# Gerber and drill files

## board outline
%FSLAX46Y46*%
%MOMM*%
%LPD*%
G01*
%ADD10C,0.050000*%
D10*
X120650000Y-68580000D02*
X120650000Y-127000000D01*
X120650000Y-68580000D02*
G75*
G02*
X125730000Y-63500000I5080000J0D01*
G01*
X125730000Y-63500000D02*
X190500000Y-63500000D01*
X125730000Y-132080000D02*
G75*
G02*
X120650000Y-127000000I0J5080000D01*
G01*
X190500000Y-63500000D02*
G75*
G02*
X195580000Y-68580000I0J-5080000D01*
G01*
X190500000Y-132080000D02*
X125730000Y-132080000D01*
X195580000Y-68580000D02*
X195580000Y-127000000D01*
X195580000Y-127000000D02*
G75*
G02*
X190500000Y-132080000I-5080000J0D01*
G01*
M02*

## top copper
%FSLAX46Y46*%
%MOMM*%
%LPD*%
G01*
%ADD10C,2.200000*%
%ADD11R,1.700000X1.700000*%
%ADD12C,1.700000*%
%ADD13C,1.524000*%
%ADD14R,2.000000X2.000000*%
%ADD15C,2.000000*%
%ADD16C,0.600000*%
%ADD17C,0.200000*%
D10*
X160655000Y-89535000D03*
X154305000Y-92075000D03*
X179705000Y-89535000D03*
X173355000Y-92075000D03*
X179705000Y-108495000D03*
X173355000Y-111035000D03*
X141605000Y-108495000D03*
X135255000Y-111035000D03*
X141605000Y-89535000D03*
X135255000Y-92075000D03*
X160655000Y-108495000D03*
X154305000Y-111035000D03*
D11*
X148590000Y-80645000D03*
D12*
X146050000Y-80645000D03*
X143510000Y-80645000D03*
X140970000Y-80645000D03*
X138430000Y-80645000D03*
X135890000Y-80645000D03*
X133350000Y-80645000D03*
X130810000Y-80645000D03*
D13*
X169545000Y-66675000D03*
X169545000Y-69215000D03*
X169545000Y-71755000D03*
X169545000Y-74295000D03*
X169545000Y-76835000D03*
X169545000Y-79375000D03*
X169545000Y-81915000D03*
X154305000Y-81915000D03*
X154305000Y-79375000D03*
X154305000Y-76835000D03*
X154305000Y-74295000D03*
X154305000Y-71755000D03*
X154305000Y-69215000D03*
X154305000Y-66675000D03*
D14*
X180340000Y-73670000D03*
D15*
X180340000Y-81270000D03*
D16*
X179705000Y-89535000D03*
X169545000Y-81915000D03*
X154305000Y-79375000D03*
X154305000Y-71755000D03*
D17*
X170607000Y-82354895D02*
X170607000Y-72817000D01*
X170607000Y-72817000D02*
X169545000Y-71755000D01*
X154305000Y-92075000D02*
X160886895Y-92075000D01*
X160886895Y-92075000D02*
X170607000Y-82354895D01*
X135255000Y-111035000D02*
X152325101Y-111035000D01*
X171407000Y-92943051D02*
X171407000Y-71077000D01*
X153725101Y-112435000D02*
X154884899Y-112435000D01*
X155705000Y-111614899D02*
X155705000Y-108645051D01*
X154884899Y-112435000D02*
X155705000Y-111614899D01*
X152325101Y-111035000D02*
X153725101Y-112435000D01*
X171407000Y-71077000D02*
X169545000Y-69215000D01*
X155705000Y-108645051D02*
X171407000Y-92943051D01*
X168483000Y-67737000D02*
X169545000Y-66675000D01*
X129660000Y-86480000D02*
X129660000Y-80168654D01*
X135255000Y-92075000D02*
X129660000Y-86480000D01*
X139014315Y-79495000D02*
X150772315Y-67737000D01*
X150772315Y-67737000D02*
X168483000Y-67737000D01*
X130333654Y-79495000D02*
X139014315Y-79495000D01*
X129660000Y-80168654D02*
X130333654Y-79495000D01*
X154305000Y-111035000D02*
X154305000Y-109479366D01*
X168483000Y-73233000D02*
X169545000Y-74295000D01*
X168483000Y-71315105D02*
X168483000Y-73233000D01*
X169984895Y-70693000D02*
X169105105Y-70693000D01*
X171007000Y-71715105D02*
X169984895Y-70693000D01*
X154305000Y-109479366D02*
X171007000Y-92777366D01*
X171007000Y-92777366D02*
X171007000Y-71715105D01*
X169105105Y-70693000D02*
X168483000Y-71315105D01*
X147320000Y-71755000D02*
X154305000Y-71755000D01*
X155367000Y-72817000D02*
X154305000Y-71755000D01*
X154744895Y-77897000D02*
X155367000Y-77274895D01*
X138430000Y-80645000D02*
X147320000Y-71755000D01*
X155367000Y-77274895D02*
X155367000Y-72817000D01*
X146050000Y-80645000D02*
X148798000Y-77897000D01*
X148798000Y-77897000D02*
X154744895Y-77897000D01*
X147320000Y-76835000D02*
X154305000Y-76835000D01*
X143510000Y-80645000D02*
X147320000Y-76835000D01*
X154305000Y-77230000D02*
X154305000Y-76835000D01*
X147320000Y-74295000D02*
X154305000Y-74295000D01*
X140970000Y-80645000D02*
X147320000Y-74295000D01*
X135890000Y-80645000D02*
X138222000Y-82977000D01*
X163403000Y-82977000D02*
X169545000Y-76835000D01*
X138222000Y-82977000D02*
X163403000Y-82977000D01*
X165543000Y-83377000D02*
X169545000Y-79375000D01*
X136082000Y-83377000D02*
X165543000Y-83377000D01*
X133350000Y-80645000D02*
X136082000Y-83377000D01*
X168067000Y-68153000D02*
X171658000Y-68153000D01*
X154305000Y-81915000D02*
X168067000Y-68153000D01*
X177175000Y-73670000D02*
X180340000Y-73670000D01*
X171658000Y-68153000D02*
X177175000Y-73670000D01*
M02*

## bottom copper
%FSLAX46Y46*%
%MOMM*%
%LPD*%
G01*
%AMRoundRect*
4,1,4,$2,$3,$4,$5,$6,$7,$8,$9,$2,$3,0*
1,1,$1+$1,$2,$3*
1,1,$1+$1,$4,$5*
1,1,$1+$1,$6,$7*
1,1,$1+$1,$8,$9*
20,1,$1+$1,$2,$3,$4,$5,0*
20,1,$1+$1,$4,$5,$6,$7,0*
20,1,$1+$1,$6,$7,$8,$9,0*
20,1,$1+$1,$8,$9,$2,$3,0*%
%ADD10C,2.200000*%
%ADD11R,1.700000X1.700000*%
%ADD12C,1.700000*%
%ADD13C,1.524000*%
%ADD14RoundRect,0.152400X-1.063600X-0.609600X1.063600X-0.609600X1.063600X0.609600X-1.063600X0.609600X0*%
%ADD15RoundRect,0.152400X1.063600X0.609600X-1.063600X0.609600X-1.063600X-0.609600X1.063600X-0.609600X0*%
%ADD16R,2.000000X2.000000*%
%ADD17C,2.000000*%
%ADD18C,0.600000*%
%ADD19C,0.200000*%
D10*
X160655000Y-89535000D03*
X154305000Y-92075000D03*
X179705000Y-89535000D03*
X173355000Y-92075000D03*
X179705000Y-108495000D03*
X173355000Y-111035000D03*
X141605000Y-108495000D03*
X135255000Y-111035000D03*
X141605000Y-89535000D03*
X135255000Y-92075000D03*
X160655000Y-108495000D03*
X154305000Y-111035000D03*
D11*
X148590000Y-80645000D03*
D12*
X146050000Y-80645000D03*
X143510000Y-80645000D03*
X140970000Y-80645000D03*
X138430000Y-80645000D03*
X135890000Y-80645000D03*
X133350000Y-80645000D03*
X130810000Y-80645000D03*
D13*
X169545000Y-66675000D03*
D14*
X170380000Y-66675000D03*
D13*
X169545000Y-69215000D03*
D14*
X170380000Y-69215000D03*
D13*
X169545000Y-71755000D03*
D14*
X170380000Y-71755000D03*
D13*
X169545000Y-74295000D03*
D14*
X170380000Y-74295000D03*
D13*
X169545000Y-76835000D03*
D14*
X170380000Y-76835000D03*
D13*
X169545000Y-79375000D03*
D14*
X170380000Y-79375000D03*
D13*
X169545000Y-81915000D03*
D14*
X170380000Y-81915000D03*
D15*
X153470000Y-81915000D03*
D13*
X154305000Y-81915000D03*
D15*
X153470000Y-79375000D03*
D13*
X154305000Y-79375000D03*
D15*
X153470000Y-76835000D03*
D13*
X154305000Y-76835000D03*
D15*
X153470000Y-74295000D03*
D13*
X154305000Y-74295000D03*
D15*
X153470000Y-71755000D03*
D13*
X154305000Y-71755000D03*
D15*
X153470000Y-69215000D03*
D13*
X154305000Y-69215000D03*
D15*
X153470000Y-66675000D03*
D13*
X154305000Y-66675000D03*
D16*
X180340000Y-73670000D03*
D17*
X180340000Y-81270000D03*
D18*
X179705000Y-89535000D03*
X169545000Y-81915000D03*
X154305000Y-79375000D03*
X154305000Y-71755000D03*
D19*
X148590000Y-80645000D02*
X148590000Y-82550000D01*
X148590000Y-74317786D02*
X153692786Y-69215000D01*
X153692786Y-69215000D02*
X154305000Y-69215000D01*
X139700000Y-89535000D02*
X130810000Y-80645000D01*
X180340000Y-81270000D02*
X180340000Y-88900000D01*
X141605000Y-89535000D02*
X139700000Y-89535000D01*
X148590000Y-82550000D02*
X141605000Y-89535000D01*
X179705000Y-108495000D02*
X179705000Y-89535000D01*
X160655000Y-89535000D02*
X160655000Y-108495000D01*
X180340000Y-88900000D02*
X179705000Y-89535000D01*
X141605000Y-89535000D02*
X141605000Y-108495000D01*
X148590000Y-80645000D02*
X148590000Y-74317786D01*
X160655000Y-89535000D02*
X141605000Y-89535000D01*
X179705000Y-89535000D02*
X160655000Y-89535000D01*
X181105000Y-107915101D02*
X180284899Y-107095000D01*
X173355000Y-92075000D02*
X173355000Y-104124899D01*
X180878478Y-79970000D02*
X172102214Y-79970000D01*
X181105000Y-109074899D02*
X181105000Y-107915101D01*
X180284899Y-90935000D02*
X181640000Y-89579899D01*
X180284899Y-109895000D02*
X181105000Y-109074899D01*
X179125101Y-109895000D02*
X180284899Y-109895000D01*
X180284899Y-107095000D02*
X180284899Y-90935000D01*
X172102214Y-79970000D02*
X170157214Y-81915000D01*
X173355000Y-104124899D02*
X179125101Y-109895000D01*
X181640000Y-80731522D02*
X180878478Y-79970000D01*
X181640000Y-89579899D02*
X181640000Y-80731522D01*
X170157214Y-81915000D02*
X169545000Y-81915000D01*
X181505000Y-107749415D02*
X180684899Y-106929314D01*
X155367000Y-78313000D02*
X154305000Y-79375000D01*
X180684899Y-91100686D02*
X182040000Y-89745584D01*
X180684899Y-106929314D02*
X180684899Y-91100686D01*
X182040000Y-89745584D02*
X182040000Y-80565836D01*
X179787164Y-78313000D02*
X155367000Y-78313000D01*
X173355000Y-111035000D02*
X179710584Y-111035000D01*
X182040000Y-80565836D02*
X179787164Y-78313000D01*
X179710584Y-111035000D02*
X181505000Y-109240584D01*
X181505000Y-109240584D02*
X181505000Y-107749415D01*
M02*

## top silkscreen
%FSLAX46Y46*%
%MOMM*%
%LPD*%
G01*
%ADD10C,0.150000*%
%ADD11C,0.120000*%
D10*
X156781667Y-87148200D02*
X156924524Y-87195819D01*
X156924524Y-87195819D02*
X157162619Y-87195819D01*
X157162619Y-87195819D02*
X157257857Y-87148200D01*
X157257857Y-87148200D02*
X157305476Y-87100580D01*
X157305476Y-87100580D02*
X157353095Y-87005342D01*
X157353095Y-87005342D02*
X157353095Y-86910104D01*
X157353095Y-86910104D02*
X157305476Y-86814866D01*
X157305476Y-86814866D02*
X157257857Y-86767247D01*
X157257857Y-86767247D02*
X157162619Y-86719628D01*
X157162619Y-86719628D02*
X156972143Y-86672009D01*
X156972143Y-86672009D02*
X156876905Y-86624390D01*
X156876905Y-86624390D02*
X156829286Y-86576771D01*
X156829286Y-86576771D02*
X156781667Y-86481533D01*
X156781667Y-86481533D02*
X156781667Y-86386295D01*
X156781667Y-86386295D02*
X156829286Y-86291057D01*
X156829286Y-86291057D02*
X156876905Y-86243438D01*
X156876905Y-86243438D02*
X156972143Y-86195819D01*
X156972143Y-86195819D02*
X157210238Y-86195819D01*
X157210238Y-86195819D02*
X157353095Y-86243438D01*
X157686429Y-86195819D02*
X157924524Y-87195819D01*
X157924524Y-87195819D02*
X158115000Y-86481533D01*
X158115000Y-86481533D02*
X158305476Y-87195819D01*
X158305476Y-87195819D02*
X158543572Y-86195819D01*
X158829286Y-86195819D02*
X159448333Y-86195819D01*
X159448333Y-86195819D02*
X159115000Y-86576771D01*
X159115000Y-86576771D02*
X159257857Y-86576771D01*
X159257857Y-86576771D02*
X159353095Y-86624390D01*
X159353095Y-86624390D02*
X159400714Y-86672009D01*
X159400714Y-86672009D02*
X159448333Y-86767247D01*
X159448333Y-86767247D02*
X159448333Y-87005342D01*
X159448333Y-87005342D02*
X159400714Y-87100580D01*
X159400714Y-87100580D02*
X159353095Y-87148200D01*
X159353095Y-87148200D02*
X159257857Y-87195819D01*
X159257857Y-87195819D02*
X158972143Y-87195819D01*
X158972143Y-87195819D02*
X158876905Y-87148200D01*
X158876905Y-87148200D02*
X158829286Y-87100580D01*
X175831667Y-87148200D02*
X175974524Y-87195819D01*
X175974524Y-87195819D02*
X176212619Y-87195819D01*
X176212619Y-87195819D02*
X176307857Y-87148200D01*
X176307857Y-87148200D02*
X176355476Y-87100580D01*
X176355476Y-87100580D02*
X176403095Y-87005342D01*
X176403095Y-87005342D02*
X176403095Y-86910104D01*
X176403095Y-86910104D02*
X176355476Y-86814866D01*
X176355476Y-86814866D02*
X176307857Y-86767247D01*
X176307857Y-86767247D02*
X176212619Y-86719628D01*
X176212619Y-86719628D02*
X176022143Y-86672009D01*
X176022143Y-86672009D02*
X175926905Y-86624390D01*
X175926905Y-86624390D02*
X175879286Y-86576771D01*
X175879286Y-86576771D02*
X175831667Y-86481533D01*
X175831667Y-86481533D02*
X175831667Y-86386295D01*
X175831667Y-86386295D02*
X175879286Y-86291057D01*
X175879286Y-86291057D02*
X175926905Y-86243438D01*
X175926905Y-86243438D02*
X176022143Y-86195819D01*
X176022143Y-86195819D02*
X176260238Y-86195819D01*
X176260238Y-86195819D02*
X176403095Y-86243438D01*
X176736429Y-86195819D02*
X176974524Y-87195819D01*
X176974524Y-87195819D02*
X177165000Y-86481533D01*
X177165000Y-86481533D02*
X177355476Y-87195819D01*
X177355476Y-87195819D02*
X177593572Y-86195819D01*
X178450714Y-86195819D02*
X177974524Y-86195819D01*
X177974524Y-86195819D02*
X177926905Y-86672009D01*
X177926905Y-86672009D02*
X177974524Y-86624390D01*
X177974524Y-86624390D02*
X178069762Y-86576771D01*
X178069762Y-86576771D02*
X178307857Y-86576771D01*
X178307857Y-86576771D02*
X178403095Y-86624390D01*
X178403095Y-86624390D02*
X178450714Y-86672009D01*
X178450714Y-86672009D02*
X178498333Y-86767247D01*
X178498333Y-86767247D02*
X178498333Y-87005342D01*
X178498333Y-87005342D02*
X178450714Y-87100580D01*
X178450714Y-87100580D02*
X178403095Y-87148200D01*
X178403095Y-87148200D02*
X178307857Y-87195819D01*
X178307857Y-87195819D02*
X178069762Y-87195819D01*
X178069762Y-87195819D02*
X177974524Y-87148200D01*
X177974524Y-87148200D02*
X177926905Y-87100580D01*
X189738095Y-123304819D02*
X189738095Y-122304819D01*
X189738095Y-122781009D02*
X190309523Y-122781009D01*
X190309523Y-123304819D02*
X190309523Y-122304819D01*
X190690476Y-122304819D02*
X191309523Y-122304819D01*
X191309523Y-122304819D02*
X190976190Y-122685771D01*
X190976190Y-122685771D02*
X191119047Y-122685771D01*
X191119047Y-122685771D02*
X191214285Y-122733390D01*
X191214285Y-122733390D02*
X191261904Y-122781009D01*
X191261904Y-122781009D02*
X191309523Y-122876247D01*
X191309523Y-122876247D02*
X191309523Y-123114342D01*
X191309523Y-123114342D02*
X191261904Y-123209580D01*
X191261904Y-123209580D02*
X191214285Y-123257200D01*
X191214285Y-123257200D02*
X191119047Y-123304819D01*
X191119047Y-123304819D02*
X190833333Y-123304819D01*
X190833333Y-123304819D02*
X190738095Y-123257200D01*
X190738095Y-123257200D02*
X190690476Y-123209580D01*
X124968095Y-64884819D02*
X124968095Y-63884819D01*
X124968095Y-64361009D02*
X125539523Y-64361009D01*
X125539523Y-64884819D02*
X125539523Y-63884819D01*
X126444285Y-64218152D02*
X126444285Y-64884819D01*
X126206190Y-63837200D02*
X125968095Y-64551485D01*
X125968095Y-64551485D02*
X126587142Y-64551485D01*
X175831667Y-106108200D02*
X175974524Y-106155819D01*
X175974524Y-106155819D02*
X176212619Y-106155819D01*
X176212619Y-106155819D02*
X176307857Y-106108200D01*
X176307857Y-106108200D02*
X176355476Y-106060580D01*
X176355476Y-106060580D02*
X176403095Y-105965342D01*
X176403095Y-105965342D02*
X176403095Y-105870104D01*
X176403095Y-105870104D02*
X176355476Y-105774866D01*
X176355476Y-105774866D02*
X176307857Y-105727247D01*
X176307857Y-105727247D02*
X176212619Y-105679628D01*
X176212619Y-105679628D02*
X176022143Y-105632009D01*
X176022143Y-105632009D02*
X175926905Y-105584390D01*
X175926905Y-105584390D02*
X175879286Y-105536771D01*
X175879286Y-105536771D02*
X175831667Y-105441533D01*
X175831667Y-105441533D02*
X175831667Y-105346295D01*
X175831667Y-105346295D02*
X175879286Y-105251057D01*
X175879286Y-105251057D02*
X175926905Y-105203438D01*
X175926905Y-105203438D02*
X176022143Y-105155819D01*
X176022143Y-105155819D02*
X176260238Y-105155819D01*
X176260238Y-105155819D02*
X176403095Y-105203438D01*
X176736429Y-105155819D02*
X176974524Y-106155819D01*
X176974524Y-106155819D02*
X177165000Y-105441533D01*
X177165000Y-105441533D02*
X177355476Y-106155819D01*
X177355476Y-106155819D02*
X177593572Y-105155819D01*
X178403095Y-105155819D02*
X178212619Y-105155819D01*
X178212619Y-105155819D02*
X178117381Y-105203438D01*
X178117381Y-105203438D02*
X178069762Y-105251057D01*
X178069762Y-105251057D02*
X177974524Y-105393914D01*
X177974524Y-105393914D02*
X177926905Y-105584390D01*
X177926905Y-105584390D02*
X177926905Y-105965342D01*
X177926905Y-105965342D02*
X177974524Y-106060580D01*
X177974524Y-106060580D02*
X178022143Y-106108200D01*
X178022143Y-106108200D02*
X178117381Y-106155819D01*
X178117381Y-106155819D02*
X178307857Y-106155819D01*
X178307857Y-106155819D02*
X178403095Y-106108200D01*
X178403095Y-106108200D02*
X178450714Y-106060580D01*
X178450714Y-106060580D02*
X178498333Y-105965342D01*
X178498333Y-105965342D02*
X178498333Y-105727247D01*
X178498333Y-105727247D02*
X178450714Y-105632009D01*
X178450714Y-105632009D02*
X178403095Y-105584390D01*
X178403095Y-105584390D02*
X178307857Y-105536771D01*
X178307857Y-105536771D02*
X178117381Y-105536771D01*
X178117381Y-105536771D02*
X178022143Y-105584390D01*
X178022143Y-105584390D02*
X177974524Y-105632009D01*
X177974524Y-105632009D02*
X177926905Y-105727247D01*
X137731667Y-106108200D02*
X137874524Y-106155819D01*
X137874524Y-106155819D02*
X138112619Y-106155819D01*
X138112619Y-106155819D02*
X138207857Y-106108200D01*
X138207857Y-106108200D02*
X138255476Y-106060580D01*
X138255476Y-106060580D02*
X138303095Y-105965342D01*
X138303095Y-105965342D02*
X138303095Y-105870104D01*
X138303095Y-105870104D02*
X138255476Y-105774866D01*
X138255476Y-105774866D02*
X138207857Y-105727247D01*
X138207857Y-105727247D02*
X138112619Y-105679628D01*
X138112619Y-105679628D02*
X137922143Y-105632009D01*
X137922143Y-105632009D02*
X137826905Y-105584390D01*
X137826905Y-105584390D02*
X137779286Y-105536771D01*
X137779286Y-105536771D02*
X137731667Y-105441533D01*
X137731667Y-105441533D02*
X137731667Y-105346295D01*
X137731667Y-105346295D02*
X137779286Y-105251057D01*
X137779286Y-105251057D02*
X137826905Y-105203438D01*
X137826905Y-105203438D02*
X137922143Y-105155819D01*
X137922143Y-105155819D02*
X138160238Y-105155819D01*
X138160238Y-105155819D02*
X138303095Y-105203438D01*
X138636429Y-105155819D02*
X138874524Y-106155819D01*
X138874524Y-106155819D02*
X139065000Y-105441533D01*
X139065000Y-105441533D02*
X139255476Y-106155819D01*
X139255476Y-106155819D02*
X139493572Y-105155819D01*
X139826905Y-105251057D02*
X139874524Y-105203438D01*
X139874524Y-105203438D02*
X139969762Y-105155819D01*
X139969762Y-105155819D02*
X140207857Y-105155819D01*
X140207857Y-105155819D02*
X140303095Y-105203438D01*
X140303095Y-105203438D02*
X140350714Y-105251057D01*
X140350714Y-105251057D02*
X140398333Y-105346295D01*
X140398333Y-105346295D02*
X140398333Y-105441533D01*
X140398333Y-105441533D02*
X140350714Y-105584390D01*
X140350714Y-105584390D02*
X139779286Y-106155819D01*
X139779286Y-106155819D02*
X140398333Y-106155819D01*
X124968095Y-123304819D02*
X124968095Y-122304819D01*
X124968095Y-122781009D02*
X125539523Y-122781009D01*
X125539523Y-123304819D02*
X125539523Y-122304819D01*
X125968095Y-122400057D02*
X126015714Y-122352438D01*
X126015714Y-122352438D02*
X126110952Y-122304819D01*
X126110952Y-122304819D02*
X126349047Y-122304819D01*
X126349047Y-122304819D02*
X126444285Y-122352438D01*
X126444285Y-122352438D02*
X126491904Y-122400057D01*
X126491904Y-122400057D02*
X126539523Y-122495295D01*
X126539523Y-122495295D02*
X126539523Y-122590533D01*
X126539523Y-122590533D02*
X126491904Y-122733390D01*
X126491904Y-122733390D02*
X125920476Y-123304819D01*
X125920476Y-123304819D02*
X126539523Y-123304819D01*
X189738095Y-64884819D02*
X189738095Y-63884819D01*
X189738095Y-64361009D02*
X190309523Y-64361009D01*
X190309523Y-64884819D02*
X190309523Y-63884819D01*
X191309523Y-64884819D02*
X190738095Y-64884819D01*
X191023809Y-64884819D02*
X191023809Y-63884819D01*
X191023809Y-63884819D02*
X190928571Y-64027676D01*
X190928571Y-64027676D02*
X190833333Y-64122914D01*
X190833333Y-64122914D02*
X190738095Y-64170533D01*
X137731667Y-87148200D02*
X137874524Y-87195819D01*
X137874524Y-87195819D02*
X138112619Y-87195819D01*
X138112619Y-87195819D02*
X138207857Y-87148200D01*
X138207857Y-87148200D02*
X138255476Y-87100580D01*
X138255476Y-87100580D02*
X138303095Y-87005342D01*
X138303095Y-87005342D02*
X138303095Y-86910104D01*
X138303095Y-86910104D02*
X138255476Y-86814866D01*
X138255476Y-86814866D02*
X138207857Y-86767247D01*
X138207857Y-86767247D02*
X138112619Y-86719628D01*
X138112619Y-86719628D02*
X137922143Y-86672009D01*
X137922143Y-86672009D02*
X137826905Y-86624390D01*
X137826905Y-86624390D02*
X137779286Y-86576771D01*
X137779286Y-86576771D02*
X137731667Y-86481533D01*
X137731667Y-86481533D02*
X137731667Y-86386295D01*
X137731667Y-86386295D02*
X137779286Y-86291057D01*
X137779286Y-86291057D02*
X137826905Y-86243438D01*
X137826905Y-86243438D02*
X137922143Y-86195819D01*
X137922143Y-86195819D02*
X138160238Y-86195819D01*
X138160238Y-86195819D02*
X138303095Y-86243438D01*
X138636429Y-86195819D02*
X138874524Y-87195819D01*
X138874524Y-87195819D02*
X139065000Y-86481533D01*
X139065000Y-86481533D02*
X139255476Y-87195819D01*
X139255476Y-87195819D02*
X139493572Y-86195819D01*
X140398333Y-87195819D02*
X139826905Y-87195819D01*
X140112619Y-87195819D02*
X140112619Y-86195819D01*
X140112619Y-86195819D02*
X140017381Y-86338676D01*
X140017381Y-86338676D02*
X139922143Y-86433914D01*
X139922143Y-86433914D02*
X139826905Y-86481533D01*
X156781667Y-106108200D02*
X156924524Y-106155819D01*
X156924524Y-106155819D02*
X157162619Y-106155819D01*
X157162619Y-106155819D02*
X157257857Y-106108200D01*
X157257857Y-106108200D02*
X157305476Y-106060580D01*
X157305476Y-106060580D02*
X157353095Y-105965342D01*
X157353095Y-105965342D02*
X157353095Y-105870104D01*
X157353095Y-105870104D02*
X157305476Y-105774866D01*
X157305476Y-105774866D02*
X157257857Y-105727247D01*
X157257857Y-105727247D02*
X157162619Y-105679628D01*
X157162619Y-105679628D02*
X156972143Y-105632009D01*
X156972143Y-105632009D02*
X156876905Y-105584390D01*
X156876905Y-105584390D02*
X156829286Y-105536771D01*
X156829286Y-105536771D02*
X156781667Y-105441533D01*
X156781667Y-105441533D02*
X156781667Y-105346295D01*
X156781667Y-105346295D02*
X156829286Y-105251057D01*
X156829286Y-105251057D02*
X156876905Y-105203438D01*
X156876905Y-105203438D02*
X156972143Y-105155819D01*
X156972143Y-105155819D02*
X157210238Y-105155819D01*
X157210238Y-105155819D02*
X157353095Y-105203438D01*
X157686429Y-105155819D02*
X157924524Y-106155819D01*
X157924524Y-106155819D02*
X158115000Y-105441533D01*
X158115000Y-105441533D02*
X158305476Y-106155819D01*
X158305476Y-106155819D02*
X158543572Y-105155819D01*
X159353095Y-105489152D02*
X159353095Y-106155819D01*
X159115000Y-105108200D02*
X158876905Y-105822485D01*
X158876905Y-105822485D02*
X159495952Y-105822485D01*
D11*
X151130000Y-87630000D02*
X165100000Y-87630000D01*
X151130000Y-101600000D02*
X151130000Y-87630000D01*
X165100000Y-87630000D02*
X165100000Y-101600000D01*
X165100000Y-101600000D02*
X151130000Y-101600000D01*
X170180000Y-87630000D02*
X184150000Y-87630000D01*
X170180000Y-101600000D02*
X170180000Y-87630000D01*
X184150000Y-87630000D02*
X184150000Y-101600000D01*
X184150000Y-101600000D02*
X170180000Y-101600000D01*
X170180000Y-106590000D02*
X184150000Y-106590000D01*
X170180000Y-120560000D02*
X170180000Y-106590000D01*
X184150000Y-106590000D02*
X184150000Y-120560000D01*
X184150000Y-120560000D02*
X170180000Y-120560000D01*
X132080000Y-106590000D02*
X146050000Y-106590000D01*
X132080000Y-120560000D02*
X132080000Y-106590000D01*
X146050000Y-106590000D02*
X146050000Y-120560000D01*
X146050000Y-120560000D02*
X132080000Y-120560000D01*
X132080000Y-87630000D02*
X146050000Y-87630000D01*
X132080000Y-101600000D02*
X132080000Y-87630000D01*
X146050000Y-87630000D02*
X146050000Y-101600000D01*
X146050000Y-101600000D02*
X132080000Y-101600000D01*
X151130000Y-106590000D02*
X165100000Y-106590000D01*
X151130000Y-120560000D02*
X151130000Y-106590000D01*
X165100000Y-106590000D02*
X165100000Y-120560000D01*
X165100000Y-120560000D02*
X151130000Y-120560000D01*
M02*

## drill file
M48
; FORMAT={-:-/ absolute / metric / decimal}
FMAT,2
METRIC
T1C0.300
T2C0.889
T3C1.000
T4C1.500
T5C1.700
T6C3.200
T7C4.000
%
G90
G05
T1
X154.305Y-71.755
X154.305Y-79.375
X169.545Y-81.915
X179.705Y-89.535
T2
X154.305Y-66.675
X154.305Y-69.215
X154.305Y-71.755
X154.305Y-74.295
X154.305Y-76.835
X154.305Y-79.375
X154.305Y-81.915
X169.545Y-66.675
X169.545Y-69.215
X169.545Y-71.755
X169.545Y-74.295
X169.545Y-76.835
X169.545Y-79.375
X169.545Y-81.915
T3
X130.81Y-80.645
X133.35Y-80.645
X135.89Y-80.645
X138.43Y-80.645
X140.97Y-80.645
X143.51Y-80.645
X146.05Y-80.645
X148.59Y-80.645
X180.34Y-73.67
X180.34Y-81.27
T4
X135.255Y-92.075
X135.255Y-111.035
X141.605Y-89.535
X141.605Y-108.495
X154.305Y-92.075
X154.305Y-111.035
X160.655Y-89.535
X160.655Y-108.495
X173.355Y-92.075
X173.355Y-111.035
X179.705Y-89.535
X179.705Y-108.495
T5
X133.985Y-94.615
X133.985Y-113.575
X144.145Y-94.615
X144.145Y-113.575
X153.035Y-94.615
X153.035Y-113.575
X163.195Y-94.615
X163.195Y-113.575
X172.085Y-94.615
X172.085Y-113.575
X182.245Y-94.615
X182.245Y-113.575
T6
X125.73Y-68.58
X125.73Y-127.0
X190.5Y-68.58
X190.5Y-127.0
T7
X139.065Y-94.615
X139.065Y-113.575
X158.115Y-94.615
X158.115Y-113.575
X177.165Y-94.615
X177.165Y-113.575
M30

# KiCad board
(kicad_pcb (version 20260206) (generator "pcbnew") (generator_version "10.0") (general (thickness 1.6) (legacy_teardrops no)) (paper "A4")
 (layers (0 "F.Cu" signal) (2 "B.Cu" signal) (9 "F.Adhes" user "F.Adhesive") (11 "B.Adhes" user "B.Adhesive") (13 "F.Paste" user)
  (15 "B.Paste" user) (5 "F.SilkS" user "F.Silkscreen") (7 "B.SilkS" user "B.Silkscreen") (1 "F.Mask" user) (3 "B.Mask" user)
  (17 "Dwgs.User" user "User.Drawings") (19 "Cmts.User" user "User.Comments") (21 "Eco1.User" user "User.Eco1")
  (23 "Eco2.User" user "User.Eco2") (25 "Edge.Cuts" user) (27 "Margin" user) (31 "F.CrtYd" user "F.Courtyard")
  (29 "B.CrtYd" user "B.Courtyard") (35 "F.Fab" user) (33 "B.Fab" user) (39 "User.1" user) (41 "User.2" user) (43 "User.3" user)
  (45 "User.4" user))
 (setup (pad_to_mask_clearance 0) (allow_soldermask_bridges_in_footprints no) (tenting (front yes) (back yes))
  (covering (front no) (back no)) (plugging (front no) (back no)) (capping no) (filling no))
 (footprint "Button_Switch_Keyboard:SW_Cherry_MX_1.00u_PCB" (layer "F.Cu") (at 160.655 89.535)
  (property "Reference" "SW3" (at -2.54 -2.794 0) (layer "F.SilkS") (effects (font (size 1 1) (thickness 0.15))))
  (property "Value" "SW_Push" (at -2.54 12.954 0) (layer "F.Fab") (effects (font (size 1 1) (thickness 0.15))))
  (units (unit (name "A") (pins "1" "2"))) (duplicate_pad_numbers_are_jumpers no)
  (fp_line (start -9.525 -1.905) (end 4.445 -1.905) (stroke (width 0.12) (type solid)) (layer "F.SilkS"))
  (fp_line (start -9.525 12.065) (end -9.525 -1.905) (stroke (width 0.12) (type solid)) (layer "F.SilkS"))
  (fp_line (start 4.445 -1.905) (end 4.445 12.065) (stroke (width 0.12) (type solid)) (layer "F.SilkS"))
  (fp_line (start 4.445 12.065) (end -9.525 12.065) (stroke (width 0.12) (type solid)) (layer "F.SilkS"))
  (pad "" np_thru_hole circle (at -7.62 5.08) (size 1.7 1.7) (drill 1.7) (layers "*.Cu" "*.Mask"))
  (pad "" np_thru_hole circle (at -2.54 5.08) (size 4 4) (drill 4) (layers "*.Cu" "*.Mask"))
  (pad "" np_thru_hole circle (at 2.54 5.08) (size 1.7 1.7) (drill 1.7) (layers "*.Cu" "*.Mask"))
  (pad "1" thru_hole circle (at 0 0) (size 2.2 2.2) (drill 1.5) (layers "*.Cu" "*.Mask") (remove_unused_layers no) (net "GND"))
  (pad "2" thru_hole circle (at -6.35 2.54) (size 2.2 2.2) (drill 1.5) (layers "*.Cu" "*.Mask") (remove_unused_layers no)
   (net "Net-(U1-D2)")))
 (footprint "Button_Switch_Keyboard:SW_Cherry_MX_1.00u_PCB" (layer "F.Cu") (at 179.705 89.535)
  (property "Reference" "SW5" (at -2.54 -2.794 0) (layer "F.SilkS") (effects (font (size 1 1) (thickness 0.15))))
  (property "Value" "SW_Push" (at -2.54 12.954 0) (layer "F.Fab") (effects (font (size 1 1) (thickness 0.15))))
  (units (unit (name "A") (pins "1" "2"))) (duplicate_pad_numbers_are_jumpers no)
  (fp_line (start -9.525 -1.905) (end 4.445 -1.905) (stroke (width 0.12) (type solid)) (layer "F.SilkS"))
  (fp_line (start -9.525 12.065) (end -9.525 -1.905) (stroke (width 0.12) (type solid)) (layer "F.SilkS"))
  (fp_line (start 4.445 -1.905) (end 4.445 12.065) (stroke (width 0.12) (type solid)) (layer "F.SilkS"))
  (fp_line (start 4.445 12.065) (end -9.525 12.065) (stroke (width 0.12) (type solid)) (layer "F.SilkS"))
  (pad "" np_thru_hole circle (at -7.62 5.08) (size 1.7 1.7) (drill 1.7) (layers "*.Cu" "*.Mask"))
  (pad "" np_thru_hole circle (at -2.54 5.08) (size 4 4) (drill 4) (layers "*.Cu" "*.Mask"))
  (pad "" np_thru_hole circle (at 2.54 5.08) (size 1.7 1.7) (drill 1.7) (layers "*.Cu" "*.Mask"))
  (pad "1" thru_hole circle (at 0 0) (size 2.2 2.2) (drill 1.5) (layers "*.Cu" "*.Mask") (remove_unused_layers no) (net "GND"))
  (pad "2" thru_hole circle (at -6.35 2.54) (size 2.2 2.2) (drill 1.5) (layers "*.Cu" "*.Mask") (remove_unused_layers no)
   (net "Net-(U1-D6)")))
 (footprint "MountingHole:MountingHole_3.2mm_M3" (layer "F.Cu") (at 190.5 127)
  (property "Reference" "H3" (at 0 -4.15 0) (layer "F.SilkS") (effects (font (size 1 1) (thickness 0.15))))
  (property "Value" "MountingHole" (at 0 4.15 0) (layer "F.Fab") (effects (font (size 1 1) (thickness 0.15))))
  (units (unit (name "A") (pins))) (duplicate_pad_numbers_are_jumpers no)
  (pad "" np_thru_hole circle (at 0 0) (size 3.2 3.2) (drill 3.2) (layers "*.Cu" "*.Mask")))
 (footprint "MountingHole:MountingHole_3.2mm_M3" (layer "F.Cu") (at 125.73 68.58)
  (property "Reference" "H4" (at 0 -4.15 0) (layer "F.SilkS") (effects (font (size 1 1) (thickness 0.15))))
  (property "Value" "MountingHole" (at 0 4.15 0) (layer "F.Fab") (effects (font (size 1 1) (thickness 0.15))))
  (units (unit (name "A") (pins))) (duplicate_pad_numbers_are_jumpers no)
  (pad "" np_thru_hole circle (at 0 0) (size 3.2 3.2) (drill 3.2) (layers "*.Cu" "*.Mask")))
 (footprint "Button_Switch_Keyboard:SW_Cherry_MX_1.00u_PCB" (layer "F.Cu") (at 179.705 108.495)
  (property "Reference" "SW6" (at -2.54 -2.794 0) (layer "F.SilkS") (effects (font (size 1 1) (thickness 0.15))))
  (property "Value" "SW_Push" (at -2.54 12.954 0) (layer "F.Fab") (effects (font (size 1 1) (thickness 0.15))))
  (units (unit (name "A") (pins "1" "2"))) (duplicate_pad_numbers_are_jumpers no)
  (fp_line (start -9.525 -1.905) (end 4.445 -1.905) (stroke (width 0.12) (type solid)) (layer "F.SilkS"))
  (fp_line (start -9.525 12.065) (end -9.525 -1.905) (stroke (width 0.12) (type solid)) (layer "F.SilkS"))
  (fp_line (start 4.445 -1.905) (end 4.445 12.065) (stroke (width 0.12) (type solid)) (layer "F.SilkS"))
  (fp_line (start 4.445 12.065) (end -9.525 12.065) (stroke (width 0.12) (type solid)) (layer "F.SilkS"))
  (pad "" np_thru_hole circle (at -7.62 5.08) (size 1.7 1.7) (drill 1.7) (layers "*.Cu" "*.Mask"))
  (pad "" np_thru_hole circle (at -2.54 5.08) (size 4 4) (drill 4) (layers "*.Cu" "*.Mask"))
  (pad "" np_thru_hole circle (at 2.54 5.08) (size 1.7 1.7) (drill 1.7) (layers "*.Cu" "*.Mask"))
  (pad "1" thru_hole circle (at 0 0) (size 2.2 2.2) (drill 1.5) (layers "*.Cu" "*.Mask") (remove_unused_layers no) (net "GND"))
  (pad "2" thru_hole circle (at -6.35 2.54) (size 2.2 2.2) (drill 1.5) (layers "*.Cu" "*.Mask") (remove_unused_layers no)
   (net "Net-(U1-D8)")))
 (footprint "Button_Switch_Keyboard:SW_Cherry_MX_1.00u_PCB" (layer "F.Cu") (at 141.605 108.495)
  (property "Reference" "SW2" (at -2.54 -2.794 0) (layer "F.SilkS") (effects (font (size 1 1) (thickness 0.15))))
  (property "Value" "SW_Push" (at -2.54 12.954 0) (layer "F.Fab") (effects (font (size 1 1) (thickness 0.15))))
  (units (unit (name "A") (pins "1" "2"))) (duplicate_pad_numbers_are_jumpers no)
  (fp_line (start -9.525 -1.905) (end 4.445 -1.905) (stroke (width 0.12) (type solid)) (layer "F.SilkS"))
  (fp_line (start -9.525 12.065) (end -9.525 -1.905) (stroke (width 0.12) (type solid)) (layer "F.SilkS"))
  (fp_line (start 4.445 -1.905) (end 4.445 12.065) (stroke (width 0.12) (type solid)) (layer "F.SilkS"))
  (fp_line (start 4.445 12.065) (end -9.525 12.065) (stroke (width 0.12) (type solid)) (layer "F.SilkS"))
  (pad "" np_thru_hole circle (at -7.62 5.08) (size 1.7 1.7) (drill 1.7) (layers "*.Cu" "*.Mask"))
  (pad "" np_thru_hole circle (at -2.54 5.08) (size 4 4) (drill 4) (layers "*.Cu" "*.Mask"))
  (pad "" np_thru_hole circle (at 2.54 5.08) (size 1.7 1.7) (drill 1.7) (layers "*.Cu" "*.Mask"))
  (pad "1" thru_hole circle (at 0 0) (size 2.2 2.2) (drill 1.5) (layers "*.Cu" "*.Mask") (remove_unused_layers no) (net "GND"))
  (pad "2" thru_hole circle (at -6.35 2.54) (size 2.2 2.2) (drill 1.5) (layers "*.Cu" "*.Mask") (remove_unused_layers no)
   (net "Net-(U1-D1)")))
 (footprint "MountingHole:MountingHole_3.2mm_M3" (layer "F.Cu") (at 125.73 127)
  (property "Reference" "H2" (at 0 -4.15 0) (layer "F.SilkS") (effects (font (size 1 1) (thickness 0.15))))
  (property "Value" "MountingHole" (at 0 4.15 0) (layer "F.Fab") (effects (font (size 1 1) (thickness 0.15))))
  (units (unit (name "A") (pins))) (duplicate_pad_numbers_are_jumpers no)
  (pad "" np_thru_hole circle (at 0 0) (size 3.2 3.2) (drill 3.2) (layers "*.Cu" "*.Mask")))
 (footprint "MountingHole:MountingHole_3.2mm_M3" (layer "F.Cu") (at 190.5 68.58)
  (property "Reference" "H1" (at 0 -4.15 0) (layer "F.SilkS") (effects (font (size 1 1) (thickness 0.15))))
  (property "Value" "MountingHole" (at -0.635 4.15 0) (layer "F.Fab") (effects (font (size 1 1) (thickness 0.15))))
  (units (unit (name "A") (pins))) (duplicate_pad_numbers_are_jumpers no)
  (pad "" np_thru_hole circle (at 0 0) (size 3.2 3.2) (drill 3.2) (layers "*.Cu" "*.Mask")))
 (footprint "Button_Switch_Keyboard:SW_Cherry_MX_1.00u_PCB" (layer "F.Cu") (at 141.605 89.535)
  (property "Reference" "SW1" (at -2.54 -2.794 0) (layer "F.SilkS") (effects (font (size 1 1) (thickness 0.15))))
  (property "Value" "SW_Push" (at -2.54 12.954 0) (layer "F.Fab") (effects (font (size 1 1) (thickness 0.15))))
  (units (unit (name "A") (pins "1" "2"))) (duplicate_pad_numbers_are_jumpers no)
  (fp_line (start -9.525 -1.905) (end 4.445 -1.905) (stroke (width 0.12) (type solid)) (layer "F.SilkS"))
  (fp_line (start -9.525 12.065) (end -9.525 -1.905) (stroke (width 0.12) (type solid)) (layer "F.SilkS"))
  (fp_line (start 4.445 -1.905) (end 4.445 12.065) (stroke (width 0.12) (type solid)) (layer "F.SilkS"))
  (fp_line (start 4.445 12.065) (end -9.525 12.065) (stroke (width 0.12) (type solid)) (layer "F.SilkS"))
  (pad "" np_thru_hole circle (at -7.62 5.08) (size 1.7 1.7) (drill 1.7) (layers "*.Cu" "*.Mask"))
  (pad "" np_thru_hole circle (at -2.54 5.08) (size 4 4) (drill 4) (layers "*.Cu" "*.Mask"))
  (pad "" np_thru_hole circle (at 2.54 5.08) (size 1.7 1.7) (drill 1.7) (layers "*.Cu" "*.Mask"))
  (pad "1" thru_hole circle (at 0 0) (size 2.2 2.2) (drill 1.5) (layers "*.Cu" "*.Mask") (remove_unused_layers no) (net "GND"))
  (pad "2" thru_hole circle (at -6.35 2.54) (size 2.2 2.2) (drill 1.5) (layers "*.Cu" "*.Mask") (remove_unused_layers no)
   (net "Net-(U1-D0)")))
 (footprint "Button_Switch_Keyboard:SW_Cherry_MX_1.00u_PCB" (layer "F.Cu") (at 160.655 108.495)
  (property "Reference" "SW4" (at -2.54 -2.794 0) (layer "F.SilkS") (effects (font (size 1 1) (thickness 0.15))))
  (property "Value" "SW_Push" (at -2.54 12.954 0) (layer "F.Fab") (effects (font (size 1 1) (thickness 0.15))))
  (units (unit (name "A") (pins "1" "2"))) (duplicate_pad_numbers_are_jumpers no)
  (fp_line (start -9.525 -1.905) (end 4.445 -1.905) (stroke (width 0.12) (type solid)) (layer "F.SilkS"))
  (fp_line (start -9.525 12.065) (end -9.525 -1.905) (stroke (width 0.12) (type solid)) (layer "F.SilkS"))
  (fp_line (start 4.445 -1.905) (end 4.445 12.065) (stroke (width 0.12) (type solid)) (layer "F.SilkS"))
  (fp_line (start 4.445 12.065) (end -9.525 12.065) (stroke (width 0.12) (type solid)) (layer "F.SilkS"))
  (pad "" np_thru_hole circle (at -7.62 5.08) (size 1.7 1.7) (drill 1.7) (layers "*.Cu" "*.Mask"))
  (pad "" np_thru_hole circle (at -2.54 5.08) (size 4 4) (drill 4) (layers "*.Cu" "*.Mask"))
  (pad "" np_thru_hole circle (at 2.54 5.08) (size 1.7 1.7) (drill 1.7) (layers "*.Cu" "*.Mask"))
  (pad "1" thru_hole circle (at 0 0) (size 2.2 2.2) (drill 1.5) (layers "*.Cu" "*.Mask") (remove_unused_layers no) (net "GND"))
  (pad "2" thru_hole circle (at -6.35 2.54) (size 2.2 2.2) (drill 1.5) (layers "*.Cu" "*.Mask") (remove_unused_layers no)
   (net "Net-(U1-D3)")))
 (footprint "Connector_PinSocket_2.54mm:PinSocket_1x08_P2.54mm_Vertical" (layer "B.Cu") (at 148.59 80.645 90)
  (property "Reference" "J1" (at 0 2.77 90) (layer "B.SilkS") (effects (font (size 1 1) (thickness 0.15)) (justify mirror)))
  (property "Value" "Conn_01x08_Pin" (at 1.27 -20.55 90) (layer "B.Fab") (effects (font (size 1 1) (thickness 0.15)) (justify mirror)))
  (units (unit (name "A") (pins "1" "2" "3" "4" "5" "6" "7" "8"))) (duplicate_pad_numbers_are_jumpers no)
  (pad "1" thru_hole rect (at 0 0 90) (size 1.7 1.7) (drill 1) (layers "*.Cu" "*.Mask") (remove_unused_layers no) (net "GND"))
  (pad "2" thru_hole circle (at 0 -2.54 90) (size 1.7 1.7) (drill 1) (layers "*.Cu" "*.Mask") (remove_unused_layers no) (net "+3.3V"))
  (pad "3" thru_hole circle (at 0 -5.08 90) (size 1.7 1.7) (drill 1) (layers "*.Cu" "*.Mask") (remove_unused_layers no)
   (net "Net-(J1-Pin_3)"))
  (pad "4" thru_hole circle (at 0 -7.62 90) (size 1.7 1.7) (drill 1) (layers "*.Cu" "*.Mask") (remove_unused_layers no)
   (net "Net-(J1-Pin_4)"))
  (pad "5" thru_hole circle (at 0 -10.16 90) (size 1.7 1.7) (drill 1) (layers "*.Cu" "*.Mask") (remove_unused_layers no) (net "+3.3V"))
  (pad "6" thru_hole circle (at 0 -12.7 90) (size 1.7 1.7) (drill 1) (layers "*.Cu" "*.Mask") (remove_unused_layers no)
   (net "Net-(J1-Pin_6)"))
  (pad "7" thru_hole circle (at 0 -15.24 90) (size 1.7 1.7) (drill 1) (layers "*.Cu" "*.Mask") (remove_unused_layers no)
   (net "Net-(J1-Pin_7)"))
  (pad "8" thru_hole circle (at 0 -17.78 90) (size 1.7 1.7) (drill 1) (layers "*.Cu" "*.Mask") (remove_unused_layers no) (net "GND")))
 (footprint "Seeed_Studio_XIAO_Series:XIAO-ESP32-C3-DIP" (layer "B.Cu") (at 161.925 74.295 90)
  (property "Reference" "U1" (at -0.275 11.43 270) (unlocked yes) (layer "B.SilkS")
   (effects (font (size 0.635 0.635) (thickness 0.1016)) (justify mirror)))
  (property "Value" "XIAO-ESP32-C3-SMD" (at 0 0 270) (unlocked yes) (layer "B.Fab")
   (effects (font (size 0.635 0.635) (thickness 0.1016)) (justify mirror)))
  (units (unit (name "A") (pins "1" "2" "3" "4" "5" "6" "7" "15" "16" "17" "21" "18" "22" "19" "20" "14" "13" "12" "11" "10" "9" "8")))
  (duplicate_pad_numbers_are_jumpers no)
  (pad "1" thru_hole circle (at 7.62 7.62) (size 1.524 1.524) (drill 0.889) (layers "*.Cu" "*.Mask") (remove_unused_layers no)
   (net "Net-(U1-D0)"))
  (pad "1" smd roundrect (at 7.62 8.455) (size 2.432 1.524) (layers "B.Cu" "B.Mask") (roundrect_rratio 0.1) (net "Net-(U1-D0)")
   (thermal_bridge_angle 45))
  (pad "2" thru_hole circle (at 5.08 7.62) (size 1.524 1.524) (drill 0.889) (layers "*.Cu" "*.Mask") (remove_unused_layers no)
   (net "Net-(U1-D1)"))
  (pad "2" smd roundrect (at 5.08 8.455) (size 2.432 1.524) (layers "B.Cu" "B.Mask") (roundrect_rratio 0.1) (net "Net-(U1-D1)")
   (thermal_bridge_angle 45))
  (pad "3" thru_hole circle (at 2.54 7.62) (size 1.524 1.524) (drill 0.889) (layers "*.Cu" "*.Mask") (remove_unused_layers no)
   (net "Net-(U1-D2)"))
  (pad "3" smd roundrect (at 2.54 8.455) (size 2.432 1.524) (layers "B.Cu" "B.Mask") (roundrect_rratio 0.1) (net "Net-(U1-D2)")
   (thermal_bridge_angle 45))
  (pad "4" thru_hole circle (at 0 7.62) (size 1.524 1.524) (drill 0.889) (layers "*.Cu" "*.Mask") (remove_unused_layers no)
   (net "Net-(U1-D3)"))
  (pad "4" smd roundrect (at 0 8.455) (size 2.432 1.524) (layers "B.Cu" "B.Mask") (roundrect_rratio 0.1) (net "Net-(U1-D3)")
   (thermal_bridge_angle 45))
  (pad "5" thru_hole circle (at -2.54 7.62) (size 1.524 1.524) (drill 0.889) (layers "*.Cu" "*.Mask") (remove_unused_layers no)
   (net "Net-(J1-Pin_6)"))
  (pad "5" smd roundrect (at -2.54 8.455) (size 2.432 1.524) (layers "B.Cu" "B.Mask") (roundrect_rratio 0.1) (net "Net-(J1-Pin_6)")
   (thermal_bridge_angle 45))
  (pad "6" thru_hole circle (at -5.08 7.62) (size 1.524 1.524) (drill 0.889) (layers "*.Cu" "*.Mask") (remove_unused_layers no)
   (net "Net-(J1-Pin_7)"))
  (pad "6" smd roundrect (at -5.08 8.455) (size 2.432 1.524) (layers "B.Cu" "B.Mask") (roundrect_rratio 0.1) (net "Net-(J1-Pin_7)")
   (thermal_bridge_angle 45))
  (pad "7" thru_hole circle (at -7.62 7.62) (size 1.524 1.524) (drill 0.889) (layers "*.Cu" "*.Mask") (remove_unused_layers no)
   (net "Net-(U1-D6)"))
  (pad "7" smd roundrect (at -7.62 8.455) (size 2.432 1.524) (layers "B.Cu" "B.Mask") (roundrect_rratio 0.1) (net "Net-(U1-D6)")
   (thermal_bridge_angle 45))
  (pad "8" smd roundrect (at -7.62 -8.455 180) (size 2.432 1.524) (layers "B.Cu" "B.Mask") (roundrect_rratio 0.1) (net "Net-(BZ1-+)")
   (thermal_bridge_angle 45))
  (pad "8" thru_hole circle (at -7.62 -7.62 180) (size 1.524 1.524) (drill 0.889) (layers "*.Cu" "*.Mask") (remove_unused_layers no)
   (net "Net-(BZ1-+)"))
  (pad "9" smd roundrect (at -5.08 -8.455 180) (size 2.432 1.524) (layers "B.Cu" "B.Mask") (roundrect_rratio 0.1) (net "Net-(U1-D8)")
   (thermal_bridge_angle 45))
  (pad "9" thru_hole circle (at -5.08 -7.62 180) (size 1.524 1.524) (drill 0.889) (layers "*.Cu" "*.Mask") (remove_unused_layers no)
   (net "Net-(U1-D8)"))
  (pad "10" smd roundrect (at -2.54 -8.455 180) (size 2.432 1.524) (layers "B.Cu" "B.Mask") (roundrect_rratio 0.1) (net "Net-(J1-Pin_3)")
   (thermal_bridge_angle 45))
  (pad "10" thru_hole circle (at -2.54 -7.62 180) (size 1.524 1.524) (drill 0.889) (layers "*.Cu" "*.Mask") (remove_unused_layers no)
   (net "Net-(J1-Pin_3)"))
  (pad "11" smd roundrect (at 0 -8.455 180) (size 2.432 1.524) (layers "B.Cu" "B.Mask") (roundrect_rratio 0.1) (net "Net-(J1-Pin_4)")
   (thermal_bridge_angle 45))
  (pad "11" thru_hole circle (at 0 -7.62 180) (size 1.524 1.524) (drill 0.889) (layers "*.Cu" "*.Mask") (remove_unused_layers no)
   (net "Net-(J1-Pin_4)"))
  (pad "12" smd roundrect (at 2.54 -8.455 180) (size 2.432 1.524) (layers "B.Cu" "B.Mask") (roundrect_rratio 0.1) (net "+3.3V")
   (thermal_bridge_angle 45))
  (pad "12" thru_hole circle (at 2.54 -7.62 180) (size 1.524 1.524) (drill 0.889) (layers "*.Cu" "*.Mask") (remove_unused_layers no)
   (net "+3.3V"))
  (pad "13" smd roundrect (at 5.08 -8.455 180) (size 2.432 1.524) (layers "B.Cu" "B.Mask") (roundrect_rratio 0.1) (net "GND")
   (thermal_bridge_angle 45))
  (pad "13" thru_hole circle (at 5.08 -7.62 180) (size 1.524 1.524) (drill 0.889) (layers "*.Cu" "*.Mask") (remove_unused_layers no)
   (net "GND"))
  (pad "14" smd roundrect (at 7.62 -8.455 180) (size 2.432 1.524) (layers "B.Cu" "B.Mask") (roundrect_rratio 0.1)
   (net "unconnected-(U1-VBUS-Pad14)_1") (thermal_bridge_angle 45))
  (pad "14" thru_hole circle (at 7.62 -7.62 180) (size 1.524 1.524) (drill 0.889) (layers "*.Cu" "*.Mask") (remove_unused_layers no)
   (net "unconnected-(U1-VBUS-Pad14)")))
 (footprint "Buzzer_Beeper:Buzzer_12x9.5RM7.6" (layer "B.Cu") (at 180.34 73.67 -90)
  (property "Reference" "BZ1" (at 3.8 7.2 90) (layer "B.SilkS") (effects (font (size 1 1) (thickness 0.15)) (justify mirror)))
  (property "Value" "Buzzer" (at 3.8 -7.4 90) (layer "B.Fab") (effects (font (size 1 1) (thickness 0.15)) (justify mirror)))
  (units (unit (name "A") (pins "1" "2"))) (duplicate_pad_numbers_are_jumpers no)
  (pad "1" thru_hole rect (at 0 0 270) (size 2 2) (drill 1) (layers "*.Cu" "*.Mask") (remove_unused_layers no) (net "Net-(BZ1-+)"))
  (pad "2" thru_hole circle (at 7.6 0 270) (size 2 2) (drill 1) (layers "*.Cu" "*.Mask") (remove_unused_layers no) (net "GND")))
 (gr_line (start 120.65 68.58) (end 120.65 127) (stroke (width 0.05) (type default)) (layer "Edge.Cuts"))
 (gr_arc (start 120.65 68.58) (mid 122.137898 64.987898) (end 125.73 63.5) (stroke (width 0.05) (type default)) (layer "Edge.Cuts"))
 (gr_line (start 125.73 63.5) (end 190.5 63.5) (stroke (width 0.05) (type default)) (layer "Edge.Cuts"))
 (gr_arc (start 125.73 132.08) (mid 122.137898 130.592102) (end 120.65 127) (stroke (width 0.05) (type default)) (layer "Edge.Cuts"))
 (gr_arc (start 190.5 63.5) (mid 194.092102 64.987898) (end 195.58 68.58) (stroke (width 0.05) (type default)) (layer "Edge.Cuts"))
 (gr_line (start 190.5 132.08) (end 125.73 132.08) (stroke (width 0.05) (type default)) (layer "Edge.Cuts"))
 (gr_line (start 195.58 68.58) (end 195.58 127) (stroke (width 0.05) (type default)) (layer "Edge.Cuts"))
 (gr_arc (start 195.58 127) (mid 194.092102 130.592102) (end 190.5 132.08) (stroke (width 0.05) (type default)) (layer "Edge.Cuts"))
 (via (at 179.705 89.535) (size 0.6) (drill 0.3) (layers "F.Cu" "B.Cu") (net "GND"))
 (segment (start 148.59 80.645) (end 148.59 82.55) (width 0.2) (layer "B.Cu") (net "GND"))
 (segment (start 148.59 74.317786) (end 153.692786 69.215) (width 0.2) (layer "B.Cu") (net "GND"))
 (segment (start 153.692786 69.215) (end 154.305 69.215) (width 0.2) (layer "B.Cu") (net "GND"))
 (segment (start 139.7 89.535) (end 130.81 80.645) (width 0.2) (layer "B.Cu") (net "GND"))
 (segment (start 180.34 81.27) (end 180.34 88.9) (width 0.2) (layer "B.Cu") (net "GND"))
 (segment (start 141.605 89.535) (end 139.7 89.535) (width 0.2) (layer "B.Cu") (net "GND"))
 (segment (start 148.59 82.55) (end 141.605 89.535) (width 0.2) (layer "B.Cu") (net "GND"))
 (segment (start 179.705 108.495) (end 179.705 89.535) (width 0.2) (layer "B.Cu") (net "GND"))
 (segment (start 160.655 89.535) (end 160.655 108.495) (width 0.2) (layer "B.Cu") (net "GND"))
 (segment (start 180.34 88.9) (end 179.705 89.535) (width 0.2) (layer "B.Cu") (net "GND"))
 (segment (start 141.605 89.535) (end 141.605 108.495) (width 0.2) (layer "B.Cu") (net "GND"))
 (segment (start 148.59 80.645) (end 148.59 74.317786) (width 0.2) (layer "B.Cu") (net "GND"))
 (segment (start 160.655 89.535) (end 141.605 89.535) (width 0.2) (layer "B.Cu") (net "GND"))
 (segment (start 179.705 89.535) (end 160.655 89.535) (width 0.2) (layer "B.Cu") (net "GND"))
 (segment (start 170.607 82.354895) (end 170.607 72.817) (width 0.2) (layer "F.Cu") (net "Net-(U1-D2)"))
 (segment (start 170.607 72.817) (end 169.545 71.755) (width 0.2) (layer "F.Cu") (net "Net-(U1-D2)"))
 (segment (start 154.305 92.075) (end 160.886895 92.075) (width 0.2) (layer "F.Cu") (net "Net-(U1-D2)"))
 (segment (start 160.886895 92.075) (end 170.607 82.354895) (width 0.2) (layer "F.Cu") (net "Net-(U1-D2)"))
 (via (at 169.545 81.915) (size 0.6) (drill 0.3) (layers "F.Cu" "B.Cu") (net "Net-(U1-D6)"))
 (segment (start 181.105 107.915101) (end 180.284899 107.095) (width 0.2) (layer "B.Cu") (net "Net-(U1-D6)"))
 (segment (start 173.355 92.075) (end 173.355 104.124899) (width 0.2) (layer "B.Cu") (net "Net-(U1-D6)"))
 (segment (start 180.878478 79.97) (end 172.102214 79.97) (width 0.2) (layer "B.Cu") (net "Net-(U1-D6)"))
 (segment (start 181.105 109.074899) (end 181.105 107.915101) (width 0.2) (layer "B.Cu") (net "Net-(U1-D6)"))
 (segment (start 180.284899 90.935) (end 181.64 89.579899) (width 0.2) (layer "B.Cu") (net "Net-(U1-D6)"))
 (segment (start 180.284899 109.895) (end 181.105 109.074899) (width 0.2) (layer "B.Cu") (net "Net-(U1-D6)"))
 (segment (start 179.125101 109.895) (end 180.284899 109.895) (width 0.2) (layer "B.Cu") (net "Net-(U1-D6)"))
 (segment (start 180.284899 107.095) (end 180.284899 90.935) (width 0.2) (layer "B.Cu") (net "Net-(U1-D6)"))
 (segment (start 172.102214 79.97) (end 170.157214 81.915) (width 0.2) (layer "B.Cu") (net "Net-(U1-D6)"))
 (segment (start 173.355 104.124899) (end 179.125101 109.895) (width 0.2) (layer "B.Cu") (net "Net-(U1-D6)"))
 (segment (start 181.64 80.731522) (end 180.878478 79.97) (width 0.2) (layer "B.Cu") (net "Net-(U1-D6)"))
 (segment (start 181.64 89.579899) (end 181.64 80.731522) (width 0.2) (layer "B.Cu") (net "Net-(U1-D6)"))
 (segment (start 170.157214 81.915) (end 169.545 81.915) (width 0.2) (layer "B.Cu") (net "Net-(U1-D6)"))
 (via (at 154.305 79.375) (size 0.6) (drill 0.3) (layers "F.Cu" "B.Cu") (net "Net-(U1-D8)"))
 (segment (start 181.505 107.749415) (end 180.684899 106.929314) (width 0.2) (layer "B.Cu") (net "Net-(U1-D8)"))
 (segment (start 155.367 78.313) (end 154.305 79.375) (width 0.2) (layer "B.Cu") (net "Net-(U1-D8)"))
 (segment (start 180.684899 91.100686) (end 182.04 89.745584) (width 0.2) (layer "B.Cu") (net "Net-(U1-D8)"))
 (segment (start 180.684899 106.929314) (end 180.684899 91.100686) (width 0.2) (layer "B.Cu") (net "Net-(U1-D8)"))
 (segment (start 182.04 89.745584) (end 182.04 80.565836) (width 0.2) (layer "B.Cu") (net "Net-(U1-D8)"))
 (segment (start 179.787164 78.313) (end 155.367 78.313) (width 0.2) (layer "B.Cu") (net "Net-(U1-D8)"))
 (segment (start 173.355 111.035) (end 179.710584 111.035) (width 0.2) (layer "B.Cu") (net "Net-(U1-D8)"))
 (segment (start 182.04 80.565836) (end 179.787164 78.313) (width 0.2) (layer "B.Cu") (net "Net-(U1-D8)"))
 (segment (start 179.710584 111.035) (end 181.505 109.240584) (width 0.2) (layer "B.Cu") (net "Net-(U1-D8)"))
 (segment (start 181.505 109.240584) (end 181.505 107.749415) (width 0.2) (layer "B.Cu") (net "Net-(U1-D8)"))
 (segment (start 135.255 111.035) (end 152.325101 111.035) (width 0.2) (layer "F.Cu") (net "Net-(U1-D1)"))
 (segment (start 171.407 92.943051) (end 171.407 71.077) (width 0.2) (layer "F.Cu") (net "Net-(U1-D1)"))
 (segment (start 153.725101 112.435) (end 154.884899 112.435) (width 0.2) (layer "F.Cu") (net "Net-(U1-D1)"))
 (segment (start 155.705 111.614899) (end 155.705 108.645051) (width 0.2) (layer "F.Cu") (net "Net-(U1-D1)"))
 (segment (start 154.884899 112.435) (end 155.705 111.614899) (width 0.2) (layer "F.Cu") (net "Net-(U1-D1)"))
 (segment (start 152.325101 111.035) (end 153.725101 112.435) (width 0.2) (layer "F.Cu") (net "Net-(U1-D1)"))
 (segment (start 171.407 71.077) (end 169.545 69.215) (width 0.2) (layer "F.Cu") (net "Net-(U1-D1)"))
 (segment (start 155.705 108.645051) (end 171.407 92.943051) (width 0.2) (layer "F.Cu") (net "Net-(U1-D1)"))
 (segment (start 168.483 67.737) (end 169.545 66.675) (width 0.2) (layer "F.Cu") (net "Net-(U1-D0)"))
 (segment (start 129.66 86.48) (end 129.66 80.168654) (width 0.2) (layer "F.Cu") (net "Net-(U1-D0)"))
 (segment (start 135.255 92.075) (end 129.66 86.48) (width 0.2) (layer "F.Cu") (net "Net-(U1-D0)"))
 (segment (start 139.014315 79.495) (end 150.772315 67.737) (width 0.2) (layer "F.Cu") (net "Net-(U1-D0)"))
 (segment (start 150.772315 67.737) (end 168.483 67.737) (width 0.2) (layer "F.Cu") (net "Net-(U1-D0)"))
 (segment (start 130.333654 79.495) (end 139.014315 79.495) (width 0.2) (layer "F.Cu") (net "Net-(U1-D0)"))
 (segment (start 129.66 80.168654) (end 130.333654 79.495) (width 0.2) (layer "F.Cu") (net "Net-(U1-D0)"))
 (segment (start 154.305 111.035) (end 154.305 109.479366) (width 0.2) (layer "F.Cu") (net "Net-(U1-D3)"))
 (segment (start 168.483 73.233) (end 169.545 74.295) (width 0.2) (layer "F.Cu") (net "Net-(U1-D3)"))
 (segment (start 168.483 71.315105) (end 168.483 73.233) (width 0.2) (layer "F.Cu") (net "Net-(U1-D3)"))
 (segment (start 169.984895 70.693) (end 169.105105 70.693) (width 0.2) (layer "F.Cu") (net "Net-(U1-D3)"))
 (segment (start 171.007 71.715105) (end 169.984895 70.693) (width 0.2) (layer "F.Cu") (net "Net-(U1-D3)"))
 (segment (start 154.305 109.479366) (end 171.007 92.777366) (width 0.2) (layer "F.Cu") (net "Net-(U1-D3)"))
 (segment (start 171.007 92.777366) (end 171.007 71.715105) (width 0.2) (layer "F.Cu") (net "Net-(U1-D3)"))
 (segment (start 169.105105 70.693) (end 168.483 71.315105) (width 0.2) (layer "F.Cu") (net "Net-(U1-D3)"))
 (segment (start 147.32 71.755) (end 154.305 71.755) (width 0.2) (layer "F.Cu") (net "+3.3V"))
 (segment (start 155.367 72.817) (end 154.305 71.755) (width 0.2) (layer "F.Cu") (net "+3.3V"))
 (segment (start 154.744895 77.897) (end 155.367 77.274895) (width 0.2) (layer "F.Cu") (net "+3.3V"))
 (segment (start 138.43 80.645) (end 147.32 71.755) (width 0.2) (layer "F.Cu") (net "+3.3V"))
 (segment (start 155.367 77.274895) (end 155.367 72.817) (width 0.2) (layer "F.Cu") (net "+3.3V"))
 (segment (start 146.05 80.645) (end 148.798 77.897) (width 0.2) (layer "F.Cu") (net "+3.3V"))
 (segment (start 148.798 77.897) (end 154.744895 77.897) (width 0.2) (layer "F.Cu") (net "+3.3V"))
 (via (at 154.305 71.755) (size 0.6) (drill 0.3) (layers "F.Cu" "B.Cu") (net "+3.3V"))
 (segment (start 147.32 76.835) (end 154.305 76.835) (width 0.2) (layer "F.Cu") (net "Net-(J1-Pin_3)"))
 (segment (start 143.51 80.645) (end 147.32 76.835) (width 0.2) (layer "F.Cu") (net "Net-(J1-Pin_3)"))
 (segment (start 154.305 77.23) (end 154.305 76.835) (width 0.2) (layer "F.Cu") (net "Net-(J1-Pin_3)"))
 (segment (start 147.32 74.295) (end 154.305 74.295) (width 0.2) (layer "F.Cu") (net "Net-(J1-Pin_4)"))
 (segment (start 140.97 80.645) (end 147.32 74.295) (width 0.2) (layer "F.Cu") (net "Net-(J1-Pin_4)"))
 (segment (start 135.89 80.645) (end 138.222 82.977) (width 0.2) (layer "F.Cu") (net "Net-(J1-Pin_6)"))
 (segment (start 163.403 82.977) (end 169.545 76.835) (width 0.2) (layer "F.Cu") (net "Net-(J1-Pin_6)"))
 (segment (start 138.222 82.977) (end 163.403 82.977) (width 0.2) (layer "F.Cu") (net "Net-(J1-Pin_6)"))
 (segment (start 165.543 83.377) (end 169.545 79.375) (width 0.2) (layer "F.Cu") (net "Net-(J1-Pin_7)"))
 (segment (start 136.082 83.377) (end 165.543 83.377) (width 0.2) (layer "F.Cu") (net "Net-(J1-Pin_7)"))
 (segment (start 133.35 80.645) (end 136.082 83.377) (width 0.2) (layer "F.Cu") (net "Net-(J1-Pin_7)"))
 (segment (start 168.067 68.153) (end 171.658 68.153) (width 0.2) (layer "F.Cu") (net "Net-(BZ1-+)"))
 (segment (start 154.305 81.915) (end 168.067 68.153) (width 0.2) (layer "F.Cu") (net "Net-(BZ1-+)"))
 (segment (start 177.175 73.67) (end 180.34 73.67) (width 0.2) (layer "F.Cu") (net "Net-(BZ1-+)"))
 (segment (start 171.658 68.153) (end 177.175 73.67) (width 0.2) (layer "F.Cu") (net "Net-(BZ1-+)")))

